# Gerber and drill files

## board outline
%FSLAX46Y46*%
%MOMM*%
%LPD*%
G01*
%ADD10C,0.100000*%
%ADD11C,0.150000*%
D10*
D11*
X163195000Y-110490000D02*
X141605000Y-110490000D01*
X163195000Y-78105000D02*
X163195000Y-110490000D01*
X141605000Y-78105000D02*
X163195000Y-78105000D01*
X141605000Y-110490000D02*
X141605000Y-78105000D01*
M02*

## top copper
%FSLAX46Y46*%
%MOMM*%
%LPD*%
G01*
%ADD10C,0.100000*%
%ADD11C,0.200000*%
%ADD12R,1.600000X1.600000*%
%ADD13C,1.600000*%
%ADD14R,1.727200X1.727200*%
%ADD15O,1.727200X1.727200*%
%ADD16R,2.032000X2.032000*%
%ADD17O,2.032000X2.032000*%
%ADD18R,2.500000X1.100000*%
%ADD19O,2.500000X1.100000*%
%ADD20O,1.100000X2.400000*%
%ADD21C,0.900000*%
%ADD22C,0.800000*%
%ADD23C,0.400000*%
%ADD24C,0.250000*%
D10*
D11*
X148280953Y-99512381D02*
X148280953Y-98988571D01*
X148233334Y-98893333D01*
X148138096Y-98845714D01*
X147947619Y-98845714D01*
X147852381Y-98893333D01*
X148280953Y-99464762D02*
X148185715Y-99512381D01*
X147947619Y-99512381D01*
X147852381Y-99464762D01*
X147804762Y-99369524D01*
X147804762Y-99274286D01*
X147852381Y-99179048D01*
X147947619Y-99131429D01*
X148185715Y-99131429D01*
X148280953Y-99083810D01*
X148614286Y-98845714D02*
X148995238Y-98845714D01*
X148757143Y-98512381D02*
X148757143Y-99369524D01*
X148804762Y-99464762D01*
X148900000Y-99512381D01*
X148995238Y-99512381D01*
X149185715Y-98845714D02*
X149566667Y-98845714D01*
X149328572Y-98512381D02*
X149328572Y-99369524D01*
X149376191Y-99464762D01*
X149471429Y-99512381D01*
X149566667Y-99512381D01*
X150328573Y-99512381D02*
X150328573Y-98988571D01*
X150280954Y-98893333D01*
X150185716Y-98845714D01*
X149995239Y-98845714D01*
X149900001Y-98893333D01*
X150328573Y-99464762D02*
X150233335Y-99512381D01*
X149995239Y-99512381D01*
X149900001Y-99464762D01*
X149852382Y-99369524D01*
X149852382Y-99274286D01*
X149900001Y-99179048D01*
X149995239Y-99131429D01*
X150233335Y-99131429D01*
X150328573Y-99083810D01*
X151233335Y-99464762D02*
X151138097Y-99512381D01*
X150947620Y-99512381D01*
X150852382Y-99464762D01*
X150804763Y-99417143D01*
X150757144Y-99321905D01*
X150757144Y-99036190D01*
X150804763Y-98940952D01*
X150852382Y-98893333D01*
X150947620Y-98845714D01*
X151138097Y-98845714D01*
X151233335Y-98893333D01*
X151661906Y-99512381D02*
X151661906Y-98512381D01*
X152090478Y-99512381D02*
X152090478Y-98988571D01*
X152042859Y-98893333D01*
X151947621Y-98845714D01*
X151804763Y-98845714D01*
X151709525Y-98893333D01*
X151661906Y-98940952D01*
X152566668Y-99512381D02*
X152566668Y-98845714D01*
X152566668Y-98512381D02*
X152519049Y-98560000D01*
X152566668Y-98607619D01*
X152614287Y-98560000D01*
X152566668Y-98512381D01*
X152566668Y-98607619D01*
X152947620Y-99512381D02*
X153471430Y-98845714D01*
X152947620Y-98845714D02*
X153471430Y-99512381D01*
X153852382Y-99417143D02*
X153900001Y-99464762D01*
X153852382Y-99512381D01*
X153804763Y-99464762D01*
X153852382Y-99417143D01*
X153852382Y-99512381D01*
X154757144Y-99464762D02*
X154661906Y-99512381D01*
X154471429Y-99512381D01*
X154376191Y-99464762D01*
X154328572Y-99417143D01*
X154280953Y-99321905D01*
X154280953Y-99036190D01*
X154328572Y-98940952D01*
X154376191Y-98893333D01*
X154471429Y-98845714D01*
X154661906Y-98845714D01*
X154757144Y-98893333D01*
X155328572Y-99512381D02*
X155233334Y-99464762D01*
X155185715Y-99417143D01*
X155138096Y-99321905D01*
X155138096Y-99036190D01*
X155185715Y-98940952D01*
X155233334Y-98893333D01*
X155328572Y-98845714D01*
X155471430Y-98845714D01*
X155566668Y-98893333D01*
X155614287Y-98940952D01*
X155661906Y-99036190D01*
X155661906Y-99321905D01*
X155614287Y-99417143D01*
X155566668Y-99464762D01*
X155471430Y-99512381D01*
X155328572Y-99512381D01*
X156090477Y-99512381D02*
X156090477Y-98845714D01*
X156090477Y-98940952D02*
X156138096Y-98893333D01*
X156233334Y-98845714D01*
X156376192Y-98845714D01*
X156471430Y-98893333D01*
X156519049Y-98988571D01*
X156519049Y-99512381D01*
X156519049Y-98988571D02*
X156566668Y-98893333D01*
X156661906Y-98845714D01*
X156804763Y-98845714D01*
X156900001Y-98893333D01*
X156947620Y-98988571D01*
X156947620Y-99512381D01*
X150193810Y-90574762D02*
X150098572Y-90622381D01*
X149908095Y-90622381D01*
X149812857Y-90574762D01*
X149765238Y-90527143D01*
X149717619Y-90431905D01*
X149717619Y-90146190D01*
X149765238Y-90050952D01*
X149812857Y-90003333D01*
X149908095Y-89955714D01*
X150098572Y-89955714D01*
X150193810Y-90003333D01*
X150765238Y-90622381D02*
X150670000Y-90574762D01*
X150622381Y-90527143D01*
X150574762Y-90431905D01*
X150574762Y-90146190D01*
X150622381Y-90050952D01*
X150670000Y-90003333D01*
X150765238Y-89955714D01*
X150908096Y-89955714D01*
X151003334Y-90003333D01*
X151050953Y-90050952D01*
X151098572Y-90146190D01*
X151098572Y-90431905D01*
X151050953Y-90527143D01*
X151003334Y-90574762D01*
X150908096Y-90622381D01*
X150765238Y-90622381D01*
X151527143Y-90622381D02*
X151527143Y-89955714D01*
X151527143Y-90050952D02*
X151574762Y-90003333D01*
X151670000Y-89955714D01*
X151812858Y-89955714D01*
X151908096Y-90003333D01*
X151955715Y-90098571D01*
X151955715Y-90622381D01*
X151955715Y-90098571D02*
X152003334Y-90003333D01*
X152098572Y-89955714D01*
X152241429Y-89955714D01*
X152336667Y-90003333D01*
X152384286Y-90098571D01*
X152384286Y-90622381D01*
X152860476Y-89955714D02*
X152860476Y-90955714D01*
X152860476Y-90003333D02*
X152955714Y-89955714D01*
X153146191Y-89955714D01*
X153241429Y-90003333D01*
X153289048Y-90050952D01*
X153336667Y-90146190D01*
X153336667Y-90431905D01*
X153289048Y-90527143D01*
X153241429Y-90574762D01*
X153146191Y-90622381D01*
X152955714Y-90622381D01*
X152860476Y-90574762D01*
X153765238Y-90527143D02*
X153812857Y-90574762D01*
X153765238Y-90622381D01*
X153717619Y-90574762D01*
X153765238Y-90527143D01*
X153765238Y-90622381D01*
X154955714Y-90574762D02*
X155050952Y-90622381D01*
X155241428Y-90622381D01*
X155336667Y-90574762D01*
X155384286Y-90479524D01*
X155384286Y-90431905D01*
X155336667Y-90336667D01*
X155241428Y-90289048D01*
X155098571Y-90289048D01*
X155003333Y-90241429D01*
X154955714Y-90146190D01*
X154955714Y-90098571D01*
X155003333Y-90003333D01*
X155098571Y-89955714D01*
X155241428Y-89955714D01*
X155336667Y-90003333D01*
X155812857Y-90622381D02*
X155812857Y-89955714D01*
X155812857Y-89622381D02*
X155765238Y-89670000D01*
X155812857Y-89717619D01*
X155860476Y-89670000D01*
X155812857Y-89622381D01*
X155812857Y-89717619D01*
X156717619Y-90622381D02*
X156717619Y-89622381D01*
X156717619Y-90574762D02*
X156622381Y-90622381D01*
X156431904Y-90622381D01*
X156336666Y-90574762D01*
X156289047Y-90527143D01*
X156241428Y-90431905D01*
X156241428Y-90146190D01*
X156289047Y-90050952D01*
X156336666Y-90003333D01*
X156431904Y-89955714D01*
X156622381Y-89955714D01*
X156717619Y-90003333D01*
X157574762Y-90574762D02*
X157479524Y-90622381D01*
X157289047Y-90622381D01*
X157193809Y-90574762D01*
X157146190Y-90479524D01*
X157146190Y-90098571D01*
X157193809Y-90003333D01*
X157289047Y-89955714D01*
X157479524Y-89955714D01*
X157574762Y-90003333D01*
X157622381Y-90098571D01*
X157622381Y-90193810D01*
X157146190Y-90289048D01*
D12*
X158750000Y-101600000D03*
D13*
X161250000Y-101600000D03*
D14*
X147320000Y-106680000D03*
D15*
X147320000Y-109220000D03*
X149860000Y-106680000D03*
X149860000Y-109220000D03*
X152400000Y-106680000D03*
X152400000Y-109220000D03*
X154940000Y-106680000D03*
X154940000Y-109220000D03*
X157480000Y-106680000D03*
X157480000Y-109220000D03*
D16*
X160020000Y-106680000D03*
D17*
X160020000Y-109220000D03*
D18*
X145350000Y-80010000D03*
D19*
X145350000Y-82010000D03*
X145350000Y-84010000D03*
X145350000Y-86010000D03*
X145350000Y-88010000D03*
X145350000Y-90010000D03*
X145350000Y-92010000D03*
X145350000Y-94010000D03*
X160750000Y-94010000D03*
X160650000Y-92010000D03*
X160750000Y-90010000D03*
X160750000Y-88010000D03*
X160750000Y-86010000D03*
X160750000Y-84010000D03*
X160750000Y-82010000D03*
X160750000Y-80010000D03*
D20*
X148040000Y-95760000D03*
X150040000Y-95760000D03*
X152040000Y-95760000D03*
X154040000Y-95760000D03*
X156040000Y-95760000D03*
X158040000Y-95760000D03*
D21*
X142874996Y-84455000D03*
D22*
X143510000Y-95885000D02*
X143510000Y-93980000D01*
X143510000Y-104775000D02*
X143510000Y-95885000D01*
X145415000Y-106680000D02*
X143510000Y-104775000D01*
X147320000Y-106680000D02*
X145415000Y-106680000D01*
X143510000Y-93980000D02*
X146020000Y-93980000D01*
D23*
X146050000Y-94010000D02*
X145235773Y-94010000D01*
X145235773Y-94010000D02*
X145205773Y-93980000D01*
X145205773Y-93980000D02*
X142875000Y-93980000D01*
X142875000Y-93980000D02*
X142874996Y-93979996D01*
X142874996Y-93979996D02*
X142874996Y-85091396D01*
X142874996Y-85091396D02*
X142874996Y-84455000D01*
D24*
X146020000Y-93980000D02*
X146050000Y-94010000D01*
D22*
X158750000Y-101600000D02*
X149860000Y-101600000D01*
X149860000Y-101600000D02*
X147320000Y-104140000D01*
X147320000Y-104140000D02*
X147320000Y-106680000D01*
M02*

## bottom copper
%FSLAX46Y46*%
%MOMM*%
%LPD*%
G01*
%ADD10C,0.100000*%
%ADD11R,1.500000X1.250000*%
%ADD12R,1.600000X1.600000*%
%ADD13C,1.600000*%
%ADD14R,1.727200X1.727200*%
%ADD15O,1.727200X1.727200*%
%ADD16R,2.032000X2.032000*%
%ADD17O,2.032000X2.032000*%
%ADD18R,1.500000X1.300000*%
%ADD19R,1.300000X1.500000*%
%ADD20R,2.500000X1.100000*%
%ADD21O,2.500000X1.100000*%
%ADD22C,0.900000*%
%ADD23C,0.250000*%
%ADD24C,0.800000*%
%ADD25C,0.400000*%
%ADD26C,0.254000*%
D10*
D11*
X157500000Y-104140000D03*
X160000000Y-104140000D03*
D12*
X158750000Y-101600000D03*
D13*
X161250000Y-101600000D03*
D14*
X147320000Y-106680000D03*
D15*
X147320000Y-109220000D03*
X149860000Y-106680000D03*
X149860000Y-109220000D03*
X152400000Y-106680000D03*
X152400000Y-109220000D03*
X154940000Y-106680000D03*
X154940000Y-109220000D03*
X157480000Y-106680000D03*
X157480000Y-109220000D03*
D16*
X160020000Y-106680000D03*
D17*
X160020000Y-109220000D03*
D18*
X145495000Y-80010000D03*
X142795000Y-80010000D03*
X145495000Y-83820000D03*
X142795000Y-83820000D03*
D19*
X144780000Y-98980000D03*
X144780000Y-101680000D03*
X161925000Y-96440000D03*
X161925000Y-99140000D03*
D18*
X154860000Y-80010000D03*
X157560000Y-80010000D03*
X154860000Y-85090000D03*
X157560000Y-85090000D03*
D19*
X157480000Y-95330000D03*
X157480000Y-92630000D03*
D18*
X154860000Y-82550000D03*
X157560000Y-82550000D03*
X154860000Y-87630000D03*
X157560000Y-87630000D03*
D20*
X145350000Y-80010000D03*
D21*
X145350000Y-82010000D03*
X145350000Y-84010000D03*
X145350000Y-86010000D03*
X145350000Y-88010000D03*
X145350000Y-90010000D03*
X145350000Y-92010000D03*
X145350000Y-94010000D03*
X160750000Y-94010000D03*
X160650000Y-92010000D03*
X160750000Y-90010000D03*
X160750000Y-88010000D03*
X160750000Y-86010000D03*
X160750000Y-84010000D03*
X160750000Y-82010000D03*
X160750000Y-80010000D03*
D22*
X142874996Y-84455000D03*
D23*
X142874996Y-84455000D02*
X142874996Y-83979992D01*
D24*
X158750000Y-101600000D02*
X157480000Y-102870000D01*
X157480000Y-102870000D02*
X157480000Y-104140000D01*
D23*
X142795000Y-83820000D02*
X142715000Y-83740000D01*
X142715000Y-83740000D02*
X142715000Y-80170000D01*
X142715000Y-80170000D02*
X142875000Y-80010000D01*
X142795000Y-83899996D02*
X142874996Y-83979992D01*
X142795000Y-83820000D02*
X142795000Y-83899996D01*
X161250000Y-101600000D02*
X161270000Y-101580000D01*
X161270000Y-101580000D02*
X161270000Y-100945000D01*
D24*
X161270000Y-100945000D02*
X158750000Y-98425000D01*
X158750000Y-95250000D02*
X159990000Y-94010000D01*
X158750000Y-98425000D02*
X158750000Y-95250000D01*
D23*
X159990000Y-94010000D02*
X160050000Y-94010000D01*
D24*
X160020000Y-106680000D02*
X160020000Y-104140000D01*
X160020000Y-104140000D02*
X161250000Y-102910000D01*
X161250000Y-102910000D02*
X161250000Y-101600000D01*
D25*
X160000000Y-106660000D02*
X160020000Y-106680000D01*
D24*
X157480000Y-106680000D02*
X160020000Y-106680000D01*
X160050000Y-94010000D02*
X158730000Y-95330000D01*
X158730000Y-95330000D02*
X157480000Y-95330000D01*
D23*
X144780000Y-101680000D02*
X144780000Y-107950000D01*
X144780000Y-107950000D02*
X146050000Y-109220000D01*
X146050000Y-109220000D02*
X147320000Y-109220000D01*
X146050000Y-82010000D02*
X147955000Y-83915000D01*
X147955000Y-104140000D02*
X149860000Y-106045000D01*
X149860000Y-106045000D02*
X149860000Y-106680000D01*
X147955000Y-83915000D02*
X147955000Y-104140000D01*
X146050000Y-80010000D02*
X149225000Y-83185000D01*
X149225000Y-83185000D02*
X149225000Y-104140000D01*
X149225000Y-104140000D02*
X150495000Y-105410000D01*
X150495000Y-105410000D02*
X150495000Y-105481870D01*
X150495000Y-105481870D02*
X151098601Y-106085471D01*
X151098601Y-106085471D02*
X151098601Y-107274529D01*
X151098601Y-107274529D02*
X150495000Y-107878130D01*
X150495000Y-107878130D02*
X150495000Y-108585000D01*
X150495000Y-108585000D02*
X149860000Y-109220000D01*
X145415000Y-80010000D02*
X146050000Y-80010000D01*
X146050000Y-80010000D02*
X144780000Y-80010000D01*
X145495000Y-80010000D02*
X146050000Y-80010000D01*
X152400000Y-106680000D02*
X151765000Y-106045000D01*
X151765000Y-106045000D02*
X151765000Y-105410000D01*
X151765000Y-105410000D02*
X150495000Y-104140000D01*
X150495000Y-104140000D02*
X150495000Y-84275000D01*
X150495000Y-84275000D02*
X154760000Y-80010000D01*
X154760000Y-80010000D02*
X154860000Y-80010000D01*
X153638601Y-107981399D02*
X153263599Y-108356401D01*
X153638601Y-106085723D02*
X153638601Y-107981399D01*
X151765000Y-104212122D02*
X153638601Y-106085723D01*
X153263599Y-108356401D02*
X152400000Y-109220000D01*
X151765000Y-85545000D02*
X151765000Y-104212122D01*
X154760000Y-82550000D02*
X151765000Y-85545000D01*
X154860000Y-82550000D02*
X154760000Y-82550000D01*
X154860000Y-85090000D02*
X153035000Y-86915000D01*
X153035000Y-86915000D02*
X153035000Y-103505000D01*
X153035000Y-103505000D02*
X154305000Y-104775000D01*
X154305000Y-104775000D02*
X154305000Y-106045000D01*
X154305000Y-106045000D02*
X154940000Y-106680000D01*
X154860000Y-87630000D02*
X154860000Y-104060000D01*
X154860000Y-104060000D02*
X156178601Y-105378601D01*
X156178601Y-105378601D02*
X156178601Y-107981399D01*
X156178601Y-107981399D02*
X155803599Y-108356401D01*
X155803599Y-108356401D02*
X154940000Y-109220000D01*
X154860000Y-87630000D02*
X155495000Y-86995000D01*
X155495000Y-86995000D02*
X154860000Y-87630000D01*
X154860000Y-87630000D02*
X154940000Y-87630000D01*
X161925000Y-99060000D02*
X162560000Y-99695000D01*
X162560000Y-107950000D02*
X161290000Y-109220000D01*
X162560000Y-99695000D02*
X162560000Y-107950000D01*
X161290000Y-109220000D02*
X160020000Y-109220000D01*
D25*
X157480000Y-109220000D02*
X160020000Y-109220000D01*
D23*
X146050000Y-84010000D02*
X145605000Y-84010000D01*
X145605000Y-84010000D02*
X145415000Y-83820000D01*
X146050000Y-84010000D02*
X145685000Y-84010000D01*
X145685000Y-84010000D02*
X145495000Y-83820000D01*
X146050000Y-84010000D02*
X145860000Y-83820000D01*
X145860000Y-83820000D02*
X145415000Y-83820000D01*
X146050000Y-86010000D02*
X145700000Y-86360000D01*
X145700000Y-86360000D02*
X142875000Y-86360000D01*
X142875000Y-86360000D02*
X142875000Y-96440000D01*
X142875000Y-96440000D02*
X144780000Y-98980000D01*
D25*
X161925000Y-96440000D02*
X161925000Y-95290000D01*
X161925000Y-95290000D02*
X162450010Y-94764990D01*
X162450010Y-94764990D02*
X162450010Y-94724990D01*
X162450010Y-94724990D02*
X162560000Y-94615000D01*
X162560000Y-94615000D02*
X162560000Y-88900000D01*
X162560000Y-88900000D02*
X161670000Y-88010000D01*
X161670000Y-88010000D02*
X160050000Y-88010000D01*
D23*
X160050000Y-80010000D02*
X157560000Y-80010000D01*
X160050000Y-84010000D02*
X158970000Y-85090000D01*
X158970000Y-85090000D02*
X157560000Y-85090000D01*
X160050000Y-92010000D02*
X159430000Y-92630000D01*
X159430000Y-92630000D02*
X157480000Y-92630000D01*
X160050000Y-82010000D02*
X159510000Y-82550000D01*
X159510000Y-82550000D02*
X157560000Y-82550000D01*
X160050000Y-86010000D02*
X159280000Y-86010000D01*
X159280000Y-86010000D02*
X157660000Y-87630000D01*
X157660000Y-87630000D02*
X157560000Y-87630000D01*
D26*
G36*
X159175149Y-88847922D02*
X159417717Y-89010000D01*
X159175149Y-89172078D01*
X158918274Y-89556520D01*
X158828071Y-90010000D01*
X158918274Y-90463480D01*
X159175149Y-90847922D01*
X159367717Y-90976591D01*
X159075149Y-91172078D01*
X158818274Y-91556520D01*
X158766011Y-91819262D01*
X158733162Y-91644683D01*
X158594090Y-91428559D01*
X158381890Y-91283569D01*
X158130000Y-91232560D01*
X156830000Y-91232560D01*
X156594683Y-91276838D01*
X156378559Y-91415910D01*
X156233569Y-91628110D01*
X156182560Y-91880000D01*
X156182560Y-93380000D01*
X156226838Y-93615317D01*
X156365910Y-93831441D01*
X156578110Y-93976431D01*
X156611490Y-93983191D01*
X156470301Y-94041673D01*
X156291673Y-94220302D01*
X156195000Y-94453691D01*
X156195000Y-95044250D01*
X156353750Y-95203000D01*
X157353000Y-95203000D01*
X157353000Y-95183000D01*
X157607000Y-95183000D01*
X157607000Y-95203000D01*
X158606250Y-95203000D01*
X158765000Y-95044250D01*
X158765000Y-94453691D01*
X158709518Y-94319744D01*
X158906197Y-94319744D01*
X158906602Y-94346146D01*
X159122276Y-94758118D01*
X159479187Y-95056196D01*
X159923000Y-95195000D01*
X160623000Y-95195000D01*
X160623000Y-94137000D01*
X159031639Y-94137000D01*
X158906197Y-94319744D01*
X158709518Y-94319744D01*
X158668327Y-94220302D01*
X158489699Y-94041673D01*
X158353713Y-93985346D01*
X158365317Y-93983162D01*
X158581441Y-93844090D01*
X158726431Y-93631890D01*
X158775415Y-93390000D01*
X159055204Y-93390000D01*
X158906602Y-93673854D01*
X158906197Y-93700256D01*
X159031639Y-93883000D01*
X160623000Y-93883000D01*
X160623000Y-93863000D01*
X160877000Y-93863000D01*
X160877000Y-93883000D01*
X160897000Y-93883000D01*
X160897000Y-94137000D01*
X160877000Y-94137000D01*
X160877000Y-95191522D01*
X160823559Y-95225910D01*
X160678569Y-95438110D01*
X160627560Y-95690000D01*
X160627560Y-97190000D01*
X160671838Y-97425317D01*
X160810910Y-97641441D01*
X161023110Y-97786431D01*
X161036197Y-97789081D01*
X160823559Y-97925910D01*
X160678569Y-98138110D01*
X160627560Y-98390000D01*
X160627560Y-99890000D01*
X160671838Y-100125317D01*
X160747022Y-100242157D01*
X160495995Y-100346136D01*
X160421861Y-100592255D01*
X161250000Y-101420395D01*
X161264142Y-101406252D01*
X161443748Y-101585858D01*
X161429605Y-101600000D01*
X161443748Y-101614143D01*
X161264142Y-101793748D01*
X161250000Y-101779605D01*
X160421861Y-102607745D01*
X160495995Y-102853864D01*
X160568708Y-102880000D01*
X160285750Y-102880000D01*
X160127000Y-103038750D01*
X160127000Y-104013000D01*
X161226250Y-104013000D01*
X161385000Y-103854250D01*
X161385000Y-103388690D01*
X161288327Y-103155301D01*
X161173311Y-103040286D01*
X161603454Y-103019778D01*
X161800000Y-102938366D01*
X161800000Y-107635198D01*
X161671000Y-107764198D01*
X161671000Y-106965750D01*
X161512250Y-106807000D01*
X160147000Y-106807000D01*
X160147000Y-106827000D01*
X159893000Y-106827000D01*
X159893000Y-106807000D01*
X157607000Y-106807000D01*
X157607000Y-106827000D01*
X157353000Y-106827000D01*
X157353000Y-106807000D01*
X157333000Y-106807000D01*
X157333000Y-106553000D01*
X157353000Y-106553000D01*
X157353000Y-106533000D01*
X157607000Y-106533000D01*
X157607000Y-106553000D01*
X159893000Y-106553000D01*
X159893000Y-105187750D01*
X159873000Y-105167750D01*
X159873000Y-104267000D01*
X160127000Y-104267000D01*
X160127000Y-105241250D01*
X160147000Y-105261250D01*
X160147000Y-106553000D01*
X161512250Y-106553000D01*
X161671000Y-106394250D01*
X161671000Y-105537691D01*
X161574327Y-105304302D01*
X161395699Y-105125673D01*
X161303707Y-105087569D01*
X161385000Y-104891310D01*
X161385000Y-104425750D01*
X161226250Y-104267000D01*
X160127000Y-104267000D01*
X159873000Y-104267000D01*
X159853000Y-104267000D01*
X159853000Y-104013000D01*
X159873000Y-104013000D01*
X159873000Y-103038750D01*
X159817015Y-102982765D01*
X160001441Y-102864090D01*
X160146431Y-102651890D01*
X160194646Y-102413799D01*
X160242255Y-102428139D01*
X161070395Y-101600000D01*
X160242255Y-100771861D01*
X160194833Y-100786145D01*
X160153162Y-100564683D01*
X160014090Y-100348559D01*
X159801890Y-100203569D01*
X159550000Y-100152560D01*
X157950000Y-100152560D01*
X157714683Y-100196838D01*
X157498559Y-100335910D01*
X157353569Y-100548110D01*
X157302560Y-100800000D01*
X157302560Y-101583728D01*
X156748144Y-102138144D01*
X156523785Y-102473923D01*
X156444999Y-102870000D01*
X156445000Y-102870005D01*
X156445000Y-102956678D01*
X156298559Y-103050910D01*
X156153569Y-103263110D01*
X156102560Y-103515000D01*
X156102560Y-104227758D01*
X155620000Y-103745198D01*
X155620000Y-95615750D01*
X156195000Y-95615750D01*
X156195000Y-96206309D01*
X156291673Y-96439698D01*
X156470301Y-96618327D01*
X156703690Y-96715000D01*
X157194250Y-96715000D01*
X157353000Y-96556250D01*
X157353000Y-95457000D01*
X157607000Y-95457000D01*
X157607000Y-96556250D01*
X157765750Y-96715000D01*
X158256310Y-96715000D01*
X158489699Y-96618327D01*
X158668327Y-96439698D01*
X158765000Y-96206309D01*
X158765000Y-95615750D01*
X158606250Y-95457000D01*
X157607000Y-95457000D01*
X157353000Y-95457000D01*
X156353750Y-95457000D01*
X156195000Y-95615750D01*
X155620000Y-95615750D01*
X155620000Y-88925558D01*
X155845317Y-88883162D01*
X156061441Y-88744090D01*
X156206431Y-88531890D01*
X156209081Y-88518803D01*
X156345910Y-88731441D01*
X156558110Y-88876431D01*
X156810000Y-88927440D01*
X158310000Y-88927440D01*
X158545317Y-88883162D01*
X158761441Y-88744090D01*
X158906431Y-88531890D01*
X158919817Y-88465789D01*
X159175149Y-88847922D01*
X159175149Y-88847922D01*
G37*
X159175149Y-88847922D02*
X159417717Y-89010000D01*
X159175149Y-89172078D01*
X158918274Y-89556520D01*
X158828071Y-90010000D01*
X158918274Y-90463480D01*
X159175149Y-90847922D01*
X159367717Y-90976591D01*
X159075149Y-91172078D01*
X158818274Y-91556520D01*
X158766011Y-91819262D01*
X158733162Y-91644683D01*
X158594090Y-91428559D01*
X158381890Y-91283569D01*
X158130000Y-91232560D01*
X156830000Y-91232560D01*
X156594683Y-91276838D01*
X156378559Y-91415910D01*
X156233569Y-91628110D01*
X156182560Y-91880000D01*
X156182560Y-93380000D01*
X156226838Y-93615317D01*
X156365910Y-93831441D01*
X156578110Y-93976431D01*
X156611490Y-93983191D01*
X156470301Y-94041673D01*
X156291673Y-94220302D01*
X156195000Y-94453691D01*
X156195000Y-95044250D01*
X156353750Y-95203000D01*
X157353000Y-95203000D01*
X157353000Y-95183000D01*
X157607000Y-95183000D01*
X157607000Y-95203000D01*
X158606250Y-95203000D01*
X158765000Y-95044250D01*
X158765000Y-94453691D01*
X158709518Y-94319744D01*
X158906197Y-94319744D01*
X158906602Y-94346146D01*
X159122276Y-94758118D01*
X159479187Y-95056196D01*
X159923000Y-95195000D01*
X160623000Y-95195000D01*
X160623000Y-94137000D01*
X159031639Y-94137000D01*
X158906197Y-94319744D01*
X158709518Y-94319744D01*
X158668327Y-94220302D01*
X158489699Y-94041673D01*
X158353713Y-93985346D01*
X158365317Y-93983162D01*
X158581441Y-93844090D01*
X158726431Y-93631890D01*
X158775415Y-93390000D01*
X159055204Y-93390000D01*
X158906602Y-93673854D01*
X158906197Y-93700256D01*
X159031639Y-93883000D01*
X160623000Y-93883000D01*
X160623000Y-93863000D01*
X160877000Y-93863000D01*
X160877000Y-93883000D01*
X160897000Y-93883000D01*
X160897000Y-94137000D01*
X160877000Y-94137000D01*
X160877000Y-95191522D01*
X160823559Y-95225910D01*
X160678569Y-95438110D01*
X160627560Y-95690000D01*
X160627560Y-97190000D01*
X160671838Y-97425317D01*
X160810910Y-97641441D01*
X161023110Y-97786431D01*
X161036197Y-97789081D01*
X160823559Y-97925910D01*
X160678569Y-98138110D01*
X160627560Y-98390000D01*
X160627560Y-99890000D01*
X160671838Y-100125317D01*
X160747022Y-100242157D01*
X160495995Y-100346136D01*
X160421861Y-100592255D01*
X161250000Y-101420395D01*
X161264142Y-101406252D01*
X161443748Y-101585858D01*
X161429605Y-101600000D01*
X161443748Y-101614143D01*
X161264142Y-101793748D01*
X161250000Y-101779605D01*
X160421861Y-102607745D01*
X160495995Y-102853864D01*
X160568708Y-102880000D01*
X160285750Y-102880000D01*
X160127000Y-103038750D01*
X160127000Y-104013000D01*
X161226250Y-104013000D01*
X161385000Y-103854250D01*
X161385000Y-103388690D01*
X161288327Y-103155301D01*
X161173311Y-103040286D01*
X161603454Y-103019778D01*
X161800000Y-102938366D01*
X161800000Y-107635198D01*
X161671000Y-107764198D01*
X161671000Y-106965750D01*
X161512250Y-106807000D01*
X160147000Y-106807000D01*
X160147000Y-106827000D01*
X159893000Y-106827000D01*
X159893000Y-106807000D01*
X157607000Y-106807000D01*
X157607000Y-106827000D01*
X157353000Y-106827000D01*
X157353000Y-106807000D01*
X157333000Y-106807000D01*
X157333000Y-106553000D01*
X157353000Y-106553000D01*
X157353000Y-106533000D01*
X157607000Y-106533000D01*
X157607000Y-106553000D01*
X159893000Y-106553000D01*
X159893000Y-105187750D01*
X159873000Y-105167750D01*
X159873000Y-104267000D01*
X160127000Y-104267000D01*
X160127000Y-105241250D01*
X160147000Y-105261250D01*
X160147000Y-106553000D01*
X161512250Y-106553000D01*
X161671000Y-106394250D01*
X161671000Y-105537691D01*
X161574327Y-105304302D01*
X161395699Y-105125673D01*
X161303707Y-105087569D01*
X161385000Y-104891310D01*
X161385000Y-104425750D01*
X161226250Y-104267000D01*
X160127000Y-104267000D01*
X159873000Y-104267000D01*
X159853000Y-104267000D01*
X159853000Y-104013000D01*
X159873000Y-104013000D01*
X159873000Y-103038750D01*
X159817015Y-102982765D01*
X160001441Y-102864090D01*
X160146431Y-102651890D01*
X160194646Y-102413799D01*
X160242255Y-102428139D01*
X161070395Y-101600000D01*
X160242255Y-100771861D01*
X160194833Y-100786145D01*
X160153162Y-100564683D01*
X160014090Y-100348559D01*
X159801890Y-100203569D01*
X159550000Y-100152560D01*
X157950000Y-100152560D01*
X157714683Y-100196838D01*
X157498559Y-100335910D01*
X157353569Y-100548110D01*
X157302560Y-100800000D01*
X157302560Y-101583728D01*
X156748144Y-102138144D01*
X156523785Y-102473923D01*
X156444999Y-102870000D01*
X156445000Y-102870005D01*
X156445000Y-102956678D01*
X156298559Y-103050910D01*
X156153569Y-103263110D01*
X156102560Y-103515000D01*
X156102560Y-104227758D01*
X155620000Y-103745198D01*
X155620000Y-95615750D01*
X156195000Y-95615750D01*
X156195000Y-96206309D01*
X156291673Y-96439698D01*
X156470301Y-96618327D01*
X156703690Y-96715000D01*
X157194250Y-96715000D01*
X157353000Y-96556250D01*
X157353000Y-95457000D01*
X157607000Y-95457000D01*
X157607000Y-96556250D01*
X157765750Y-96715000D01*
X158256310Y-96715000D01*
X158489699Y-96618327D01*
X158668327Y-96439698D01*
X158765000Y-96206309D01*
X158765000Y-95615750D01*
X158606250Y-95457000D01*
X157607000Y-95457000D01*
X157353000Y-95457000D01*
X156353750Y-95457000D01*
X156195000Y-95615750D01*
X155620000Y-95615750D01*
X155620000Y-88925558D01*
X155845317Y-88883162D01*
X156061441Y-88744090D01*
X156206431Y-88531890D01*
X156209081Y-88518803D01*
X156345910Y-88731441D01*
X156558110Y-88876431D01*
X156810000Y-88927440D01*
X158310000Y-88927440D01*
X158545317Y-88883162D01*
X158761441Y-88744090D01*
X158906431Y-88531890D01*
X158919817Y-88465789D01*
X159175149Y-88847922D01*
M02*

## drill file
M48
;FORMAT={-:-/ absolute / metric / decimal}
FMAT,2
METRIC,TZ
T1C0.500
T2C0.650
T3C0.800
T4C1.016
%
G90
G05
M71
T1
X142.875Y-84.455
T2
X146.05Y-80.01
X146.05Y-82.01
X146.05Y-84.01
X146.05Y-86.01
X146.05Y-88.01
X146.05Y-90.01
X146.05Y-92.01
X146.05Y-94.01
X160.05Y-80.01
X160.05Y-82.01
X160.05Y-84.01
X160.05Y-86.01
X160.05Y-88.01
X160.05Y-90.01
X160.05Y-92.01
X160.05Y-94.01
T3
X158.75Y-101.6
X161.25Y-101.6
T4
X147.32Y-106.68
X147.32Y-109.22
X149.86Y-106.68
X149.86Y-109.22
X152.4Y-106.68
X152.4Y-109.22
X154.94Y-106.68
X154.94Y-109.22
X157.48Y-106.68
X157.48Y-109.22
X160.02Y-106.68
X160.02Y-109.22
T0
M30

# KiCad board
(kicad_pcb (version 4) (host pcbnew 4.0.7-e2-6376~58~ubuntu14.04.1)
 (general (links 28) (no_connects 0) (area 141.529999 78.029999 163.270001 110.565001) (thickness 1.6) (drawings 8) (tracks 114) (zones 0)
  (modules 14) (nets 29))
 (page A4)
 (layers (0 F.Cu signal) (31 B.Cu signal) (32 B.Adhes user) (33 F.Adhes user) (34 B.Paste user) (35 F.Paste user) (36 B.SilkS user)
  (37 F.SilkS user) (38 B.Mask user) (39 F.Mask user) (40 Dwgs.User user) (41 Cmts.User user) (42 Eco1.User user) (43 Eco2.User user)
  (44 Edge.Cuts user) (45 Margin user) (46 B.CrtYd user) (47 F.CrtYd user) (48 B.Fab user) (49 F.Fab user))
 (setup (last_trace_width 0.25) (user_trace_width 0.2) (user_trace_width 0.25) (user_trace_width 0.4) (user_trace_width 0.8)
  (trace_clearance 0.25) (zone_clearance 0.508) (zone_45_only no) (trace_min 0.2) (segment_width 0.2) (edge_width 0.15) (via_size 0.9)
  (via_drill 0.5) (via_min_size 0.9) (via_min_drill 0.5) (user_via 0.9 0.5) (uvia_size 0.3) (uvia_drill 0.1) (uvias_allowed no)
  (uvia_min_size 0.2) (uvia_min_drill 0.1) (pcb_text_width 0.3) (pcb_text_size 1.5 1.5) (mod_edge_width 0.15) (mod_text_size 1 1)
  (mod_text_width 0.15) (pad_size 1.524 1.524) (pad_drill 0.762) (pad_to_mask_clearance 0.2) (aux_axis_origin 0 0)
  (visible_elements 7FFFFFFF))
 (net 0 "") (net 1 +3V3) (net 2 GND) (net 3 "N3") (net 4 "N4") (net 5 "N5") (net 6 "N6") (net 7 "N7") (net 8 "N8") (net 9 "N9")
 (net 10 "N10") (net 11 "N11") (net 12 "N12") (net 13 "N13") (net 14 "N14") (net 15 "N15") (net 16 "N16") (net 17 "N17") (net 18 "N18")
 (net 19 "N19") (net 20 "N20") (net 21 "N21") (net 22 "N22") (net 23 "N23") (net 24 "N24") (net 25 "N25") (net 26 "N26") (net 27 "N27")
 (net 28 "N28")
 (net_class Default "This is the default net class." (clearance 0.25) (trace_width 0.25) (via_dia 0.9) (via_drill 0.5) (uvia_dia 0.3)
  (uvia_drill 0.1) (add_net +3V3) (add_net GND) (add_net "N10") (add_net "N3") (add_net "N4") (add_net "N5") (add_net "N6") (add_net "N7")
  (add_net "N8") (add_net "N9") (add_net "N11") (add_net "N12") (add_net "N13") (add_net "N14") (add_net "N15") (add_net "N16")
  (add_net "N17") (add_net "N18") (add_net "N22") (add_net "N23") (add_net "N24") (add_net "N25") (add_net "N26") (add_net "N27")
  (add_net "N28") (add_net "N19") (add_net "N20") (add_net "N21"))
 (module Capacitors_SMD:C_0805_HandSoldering (layer B.Cu) (at 158.75 104.14)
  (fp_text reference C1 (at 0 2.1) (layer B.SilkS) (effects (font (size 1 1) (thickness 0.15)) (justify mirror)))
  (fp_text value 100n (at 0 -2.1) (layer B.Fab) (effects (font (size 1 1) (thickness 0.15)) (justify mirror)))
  (pad 1 smd rect (at -1.25 0) (size 1.5 1.25) (layers B.Cu B.Paste B.Mask) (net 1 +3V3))
  (pad 2 smd rect (at 1.25 0) (size 1.5 1.25) (layers B.Cu B.Paste B.Mask) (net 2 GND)))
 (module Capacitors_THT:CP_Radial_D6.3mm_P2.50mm (layer F.Cu) (at 158.75 101.6)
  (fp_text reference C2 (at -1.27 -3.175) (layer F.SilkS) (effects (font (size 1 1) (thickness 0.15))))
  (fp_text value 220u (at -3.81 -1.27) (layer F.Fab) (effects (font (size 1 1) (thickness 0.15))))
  (pad 1 thru_hole rect (at 0 0) (size 1.6 1.6) (drill 0.8) (layers *.Cu *.Mask) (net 1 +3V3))
  (pad 2 thru_hole circle (at 2.5 0) (size 1.6 1.6) (drill 0.8) (layers *.Cu *.Mask) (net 2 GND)))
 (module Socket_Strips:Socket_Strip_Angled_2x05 (layer F.Cu) (at 147.32 106.68)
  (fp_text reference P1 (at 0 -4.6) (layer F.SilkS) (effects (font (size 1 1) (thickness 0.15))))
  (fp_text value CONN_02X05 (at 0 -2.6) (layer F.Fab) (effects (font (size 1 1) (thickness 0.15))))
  (pad 1 thru_hole rect (at 0 0) (size 1.7272 1.7272) (drill 1.016) (layers *.Cu *.Mask) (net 1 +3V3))
  (pad 2 thru_hole oval (at 0 2.54) (size 1.7272 1.7272) (drill 1.016) (layers *.Cu *.Mask) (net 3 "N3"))
  (pad 3 thru_hole oval (at 2.54 0) (size 1.7272 1.7272) (drill 1.016) (layers *.Cu *.Mask) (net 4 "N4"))
  (pad 4 thru_hole oval (at 2.54 2.54) (size 1.7272 1.7272) (drill 1.016) (layers *.Cu *.Mask) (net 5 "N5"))
  (pad 5 thru_hole oval (at 5.08 0) (size 1.7272 1.7272) (drill 1.016) (layers *.Cu *.Mask) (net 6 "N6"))
  (pad 6 thru_hole oval (at 5.08 2.54) (size 1.7272 1.7272) (drill 1.016) (layers *.Cu *.Mask) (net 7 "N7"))
  (pad 7 thru_hole oval (at 7.62 0) (size 1.7272 1.7272) (drill 1.016) (layers *.Cu *.Mask) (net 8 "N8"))
  (pad 8 thru_hole oval (at 7.62 2.54) (size 1.7272 1.7272) (drill 1.016) (layers *.Cu *.Mask) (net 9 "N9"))
  (pad 9 thru_hole oval (at 10.16 0) (size 1.7272 1.7272) (drill 1.016) (layers *.Cu *.Mask) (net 2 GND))
  (pad 10 thru_hole oval (at 10.16 2.54) (size 1.7272 1.7272) (drill 1.016) (layers *.Cu *.Mask) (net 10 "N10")))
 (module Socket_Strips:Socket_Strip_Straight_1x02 (layer F.Cu) (at 160.02 106.68 270)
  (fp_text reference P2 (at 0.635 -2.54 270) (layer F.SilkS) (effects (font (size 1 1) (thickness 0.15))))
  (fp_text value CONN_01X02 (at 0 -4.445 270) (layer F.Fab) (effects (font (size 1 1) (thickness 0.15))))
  (pad 1 thru_hole rect (at 0 0 270) (size 2.032 2.032) (drill 1.016) (layers *.Cu *.Mask) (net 2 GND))
  (pad 2 thru_hole oval (at 2.54 0 270) (size 2.032 2.032) (drill 1.016) (layers *.Cu *.Mask) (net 10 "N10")))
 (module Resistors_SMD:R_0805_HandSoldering (layer B.Cu) (at 144.145 80.01 180)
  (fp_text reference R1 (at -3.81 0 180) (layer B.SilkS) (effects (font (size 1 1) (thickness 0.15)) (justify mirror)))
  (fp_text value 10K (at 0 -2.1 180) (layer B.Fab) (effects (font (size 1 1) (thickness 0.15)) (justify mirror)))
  (pad 1 smd rect (at -1.35 0 180) (size 1.5 1.3) (layers B.Cu B.Paste B.Mask) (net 5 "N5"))
  (pad 2 smd rect (at 1.35 0 180) (size 1.5 1.3) (layers B.Cu B.Paste B.Mask) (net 1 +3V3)))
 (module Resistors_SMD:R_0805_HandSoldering (layer B.Cu) (at 144.145 83.82 180)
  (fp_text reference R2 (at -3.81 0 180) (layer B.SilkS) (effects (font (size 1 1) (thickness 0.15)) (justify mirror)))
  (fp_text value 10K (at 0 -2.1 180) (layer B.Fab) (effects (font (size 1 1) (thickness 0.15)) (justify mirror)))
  (pad 1 smd rect (at -1.35 0 180) (size 1.5 1.3) (layers B.Cu B.Paste B.Mask) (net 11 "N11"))
  (pad 2 smd rect (at 1.35 0 180) (size 1.5 1.3) (layers B.Cu B.Paste B.Mask) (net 1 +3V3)))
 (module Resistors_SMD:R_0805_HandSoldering (layer B.Cu) (at 144.78 100.33 270)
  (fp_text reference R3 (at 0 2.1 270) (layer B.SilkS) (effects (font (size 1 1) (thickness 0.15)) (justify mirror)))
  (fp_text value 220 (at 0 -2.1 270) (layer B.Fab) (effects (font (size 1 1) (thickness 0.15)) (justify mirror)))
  (pad 1 smd rect (at -1.35 0 270) (size 1.5 1.3) (layers B.Cu B.Paste B.Mask) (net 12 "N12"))
  (pad 2 smd rect (at 1.35 0 270) (size 1.5 1.3) (layers B.Cu B.Paste B.Mask) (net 3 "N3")))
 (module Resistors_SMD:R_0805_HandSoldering (layer B.Cu) (at 161.925 97.79 270)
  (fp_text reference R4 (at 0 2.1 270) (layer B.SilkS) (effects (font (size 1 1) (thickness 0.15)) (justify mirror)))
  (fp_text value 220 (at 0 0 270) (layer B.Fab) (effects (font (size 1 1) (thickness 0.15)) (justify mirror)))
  (pad 1 smd rect (at -1.35 0 270) (size 1.5 1.3) (layers B.Cu B.Paste B.Mask) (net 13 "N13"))
  (pad 2 smd rect (at 1.35 0 270) (size 1.5 1.3) (layers B.Cu B.Paste B.Mask) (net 10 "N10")))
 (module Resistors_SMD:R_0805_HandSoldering (layer B.Cu) (at 156.21 80.01)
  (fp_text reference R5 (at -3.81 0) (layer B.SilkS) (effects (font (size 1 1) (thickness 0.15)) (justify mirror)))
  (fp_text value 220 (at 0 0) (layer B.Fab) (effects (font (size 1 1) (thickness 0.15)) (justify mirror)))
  (pad 1 smd rect (at -1.35 0) (size 1.5 1.3) (layers B.Cu B.Paste B.Mask) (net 6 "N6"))
  (pad 2 smd rect (at 1.35 0) (size 1.5 1.3) (layers B.Cu B.Paste B.Mask) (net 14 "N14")))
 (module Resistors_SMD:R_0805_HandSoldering (layer B.Cu) (at 156.21 85.09)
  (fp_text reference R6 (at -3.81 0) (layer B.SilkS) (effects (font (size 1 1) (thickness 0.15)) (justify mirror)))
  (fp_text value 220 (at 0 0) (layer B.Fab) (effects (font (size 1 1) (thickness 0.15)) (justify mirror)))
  (pad 1 smd rect (at -1.35 0) (size 1.5 1.3) (layers B.Cu B.Paste B.Mask) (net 8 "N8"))
  (pad 2 smd rect (at 1.35 0) (size 1.5 1.3) (layers B.Cu B.Paste B.Mask) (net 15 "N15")))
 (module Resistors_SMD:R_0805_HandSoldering (layer B.Cu) (at 157.48 93.98 90)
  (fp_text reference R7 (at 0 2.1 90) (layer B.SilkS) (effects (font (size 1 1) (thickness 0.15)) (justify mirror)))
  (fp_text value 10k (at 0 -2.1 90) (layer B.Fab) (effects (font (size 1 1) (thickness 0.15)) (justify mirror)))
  (pad 1 smd rect (at -1.35 0 90) (size 1.5 1.3) (layers B.Cu B.Paste B.Mask) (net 2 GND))
  (pad 2 smd rect (at 1.35 0 90) (size 1.5 1.3) (layers B.Cu B.Paste B.Mask) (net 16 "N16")))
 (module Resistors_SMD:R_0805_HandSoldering (layer B.Cu) (at 156.21 82.55)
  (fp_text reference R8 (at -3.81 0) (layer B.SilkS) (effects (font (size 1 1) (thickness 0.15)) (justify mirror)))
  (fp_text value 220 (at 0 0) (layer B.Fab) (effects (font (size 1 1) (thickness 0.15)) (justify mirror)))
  (pad 1 smd rect (at -1.35 0) (size 1.5 1.3) (layers B.Cu B.Paste B.Mask) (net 7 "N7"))
  (pad 2 smd rect (at 1.35 0) (size 1.5 1.3) (layers B.Cu B.Paste B.Mask) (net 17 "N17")))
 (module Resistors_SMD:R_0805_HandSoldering (layer B.Cu) (at 156.21 87.63)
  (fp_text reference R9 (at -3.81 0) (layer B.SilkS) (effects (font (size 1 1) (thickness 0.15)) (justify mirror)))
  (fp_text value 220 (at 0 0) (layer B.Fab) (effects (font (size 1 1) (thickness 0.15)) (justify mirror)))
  (pad 1 smd rect (at -1.35 0) (size 1.5 1.3) (layers B.Cu B.Paste B.Mask) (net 9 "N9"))
  (pad 2 smd rect (at 1.35 0) (size 1.5 1.3) (layers B.Cu B.Paste B.Mask) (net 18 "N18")))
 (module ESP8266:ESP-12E (layer F.Cu) (at 146.05 80.01)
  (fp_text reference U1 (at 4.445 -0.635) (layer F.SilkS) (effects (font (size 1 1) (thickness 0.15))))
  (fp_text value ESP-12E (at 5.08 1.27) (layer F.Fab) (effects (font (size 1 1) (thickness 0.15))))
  (pad 1 thru_hole rect (at 0 0) (size 2.5 1.1) (drill 0.65 (offset -0.7 0)) (layers *.Cu *.Mask F.SilkS) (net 5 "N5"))
  (pad 2 thru_hole oval (at 0 2) (size 2.5 1.1) (drill 0.65 (offset -0.7 0)) (layers *.Cu *.Mask F.SilkS) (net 4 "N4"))
  (pad 3 thru_hole oval (at 0 4) (size 2.5 1.1) (drill 0.65 (offset -0.7 0)) (layers *.Cu *.Mask F.SilkS) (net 11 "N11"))
  (pad 4 thru_hole oval (at 0 6) (size 2.5 1.1) (drill 0.65 (offset -0.7 0)) (layers *.Cu *.Mask F.SilkS) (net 12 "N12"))
  (pad 5 thru_hole oval (at 0 8) (size 2.5 1.1) (drill 0.65 (offset -0.7 0)) (layers *.Cu *.Mask F.SilkS) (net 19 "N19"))
  (pad 6 thru_hole oval (at 0 10) (size 2.5 1.1) (drill 0.65 (offset -0.7 0)) (layers *.Cu *.Mask F.SilkS) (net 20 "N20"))
  (pad 7 thru_hole oval (at 0 12) (size 2.5 1.1) (drill 0.65 (offset -0.7 0)) (layers *.Cu *.Mask F.SilkS) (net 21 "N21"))
  (pad 8 thru_hole oval (at 0 14) (size 2.5 1.1) (drill 0.65 (offset -0.7 0)) (layers *.Cu *.Mask F.SilkS) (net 1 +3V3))
  (pad 9 thru_hole oval (at 14 14) (size 2.5 1.1) (drill 0.65 (offset 0.7 0)) (layers *.Cu *.Mask F.SilkS) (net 2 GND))
  (pad 10 thru_hole oval (at 14 12) (size 2.5 1.1) (drill 0.65 (offset 0.6 0)) (layers *.Cu *.Mask F.SilkS) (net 16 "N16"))
  (pad 11 thru_hole oval (at 14 10) (size 2.5 1.1) (drill 0.65 (offset 0.7 0)) (layers *.Cu *.Mask F.SilkS) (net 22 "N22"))
  (pad 12 thru_hole oval (at 14 8) (size 2.5 1.1) (drill 0.65 (offset 0.7 0)) (layers *.Cu *.Mask F.SilkS) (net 13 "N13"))
  (pad 13 thru_hole oval (at 14 6) (size 2.5 1.1) (drill 0.65 (offset 0.7 0)) (layers *.Cu *.Mask F.SilkS) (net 18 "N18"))
  (pad 14 thru_hole oval (at 14 4) (size 2.5 1.1) (drill 0.65 (offset 0.7 0)) (layers *.Cu *.Mask F.SilkS) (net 15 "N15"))
  (pad 15 thru_hole oval (at 14 2) (size 2.5 1.1) (drill 0.65 (offset 0.7 0)) (layers *.Cu *.Mask F.SilkS) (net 17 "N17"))
  (pad 16 thru_hole oval (at 14 0) (size 2.5 1.1) (drill 0.65 (offset 0.7 0)) (layers *.Cu *.Mask F.SilkS) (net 14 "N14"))
  (pad 17 smd oval (at 1.99 15.75 90) (size 2.4 1.1) (layers F.Cu F.Paste F.Mask) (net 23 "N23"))
  (pad 18 smd oval (at 3.99 15.75 90) (size 2.4 1.1) (layers F.Cu F.Paste F.Mask) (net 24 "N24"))
  (pad 19 smd oval (at 5.99 15.75 90) (size 2.4 1.1) (layers F.Cu F.Paste F.Mask) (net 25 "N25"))
  (pad 20 smd oval (at 7.99 15.75 90) (size 2.4 1.1) (layers F.Cu F.Paste F.Mask) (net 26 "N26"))
  (pad 21 smd oval (at 9.99 15.75 90) (size 2.4 1.1) (layers F.Cu F.Paste F.Mask) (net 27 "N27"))
  (pad 22 smd oval (at 11.99 15.75 90) (size 2.4 1.1) (layers F.Cu F.Paste F.Mask) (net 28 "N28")))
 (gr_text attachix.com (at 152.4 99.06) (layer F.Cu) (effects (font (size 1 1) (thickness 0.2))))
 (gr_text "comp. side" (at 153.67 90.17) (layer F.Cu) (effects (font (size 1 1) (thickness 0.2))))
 (gr_line (start 163.195 110.49) (end 141.605 110.49) (angle 90) (layer Edge.Cuts) (width 0.15))
 (gr_line (start 163.195 78.105) (end 163.195 110.49) (angle 90) (layer Edge.Cuts) (width 0.15))
 (gr_line (start 141.605 78.105) (end 163.195 78.105) (angle 90) (layer Edge.Cuts) (width 0.15))
 (gr_line (start 141.605 110.49) (end 141.605 78.105) (angle 90) (layer Edge.Cuts) (width 0.15))
 (segment (start 143.51 95.885) (end 143.51 93.98) (width 0.8) (layer F.Cu) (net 1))
 (segment (start 143.51 104.775) (end 143.51 95.885) (width 0.8) (layer F.Cu) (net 1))
 (segment (start 145.415 106.68) (end 143.51 104.775) (width 0.8) (layer F.Cu) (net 1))
 (segment (start 147.32 106.68) (end 145.415 106.68) (width 0.8) (layer F.Cu) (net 1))
 (segment (start 143.51 93.98) (end 146.02 93.98) (width 0.8) (layer F.Cu) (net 1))
 (segment (start 146.05 94.01) (end 145.235773 94.01) (width 0.4) (layer F.Cu) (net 1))
 (segment (start 145.235773 94.01) (end 145.205773 93.98) (width 0.4) (layer F.Cu) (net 1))
 (segment (start 145.205773 93.98) (end 142.875 93.98) (width 0.4) (layer F.Cu) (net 1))
 (segment (start 142.875 93.98) (end 142.874996 93.979996) (width 0.4) (layer F.Cu) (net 1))
 (segment (start 142.874996 93.979996) (end 142.874996 85.091396) (width 0.4) (layer F.Cu) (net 1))
 (segment (start 142.874996 85.091396) (end 142.874996 84.455) (width 0.4) (layer F.Cu) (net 1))
 (segment (start 146.02 93.98) (end 146.05 94.01) (width 0.25) (layer F.Cu) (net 1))
 (via (at 142.874996 84.455) (size 0.9) (drill 0.5) (layers F.Cu B.Cu) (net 1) (status 30))
 (segment (start 142.874996 84.455) (end 142.874996 83.979992) (width 0.25) (layer B.Cu) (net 1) (status 30))
 (segment (start 158.75 101.6) (end 149.86 101.6) (width 0.8) (layer F.Cu) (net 1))
 (segment (start 149.86 101.6) (end 147.32 104.14) (width 0.8) (layer F.Cu) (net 1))
 (segment (start 147.32 104.14) (end 147.32 106.68) (width 0.8) (layer F.Cu) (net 1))
 (segment (start 158.75 101.6) (end 157.48 102.87) (width 0.8) (layer B.Cu) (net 1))
 (segment (start 157.48 102.87) (end 157.48 104.14) (width 0.8) (layer B.Cu) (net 1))
 (segment (start 142.795 83.82) (end 142.715 83.74) (width 0.25) (layer B.Cu) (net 1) (status 30))
 (segment (start 142.715 83.74) (end 142.715 80.17) (width 0.25) (layer B.Cu) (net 1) (status 20))
 (segment (start 142.715 80.17) (end 142.875 80.01) (width 0.25) (layer B.Cu) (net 1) (status 30))
 (segment (start 142.795 83.899996) (end 142.874996 83.979992) (width 0.25) (layer B.Cu) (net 1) (status 30))
 (segment (start 142.795 83.82) (end 142.795 83.899996) (width 0.25) (layer B.Cu) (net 1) (status 30))
 (segment (start 161.25 101.6) (end 161.27 101.58) (width 0.25) (layer B.Cu) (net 2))
 (segment (start 161.27 101.58) (end 161.27 100.945) (width 0.25) (layer B.Cu) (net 2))
 (segment (start 161.27 100.945) (end 158.75 98.425) (width 0.8) (layer B.Cu) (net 2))
 (segment (start 158.75 95.25) (end 159.99 94.01) (width 0.8) (layer B.Cu) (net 2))
 (segment (start 158.75 98.425) (end 158.75 95.25) (width 0.8) (layer B.Cu) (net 2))
 (segment (start 159.99 94.01) (end 160.05 94.01) (width 0.25) (layer B.Cu) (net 2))
 (segment (start 160.02 106.68) (end 160.02 104.14) (width 0.8) (layer B.Cu) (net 2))
 (segment (start 160.02 104.14) (end 161.25 102.91) (width 0.8) (layer B.Cu) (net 2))
 (segment (start 161.25 102.91) (end 161.25 101.6) (width 0.8) (layer B.Cu) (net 2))
 (segment (start 160 106.66) (end 160.02 106.68) (width 0.4) (layer B.Cu) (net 2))
 (segment (start 157.48 106.68) (end 160.02 106.68) (width 0.8) (layer B.Cu) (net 2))
 (segment (start 160.05 94.01) (end 158.73 95.33) (width 0.8) (layer B.Cu) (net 2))
 (segment (start 158.73 95.33) (end 157.48 95.33) (width 0.8) (layer B.Cu) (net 2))
 (segment (start 144.78 101.68) (end 144.78 107.95) (width 0.25) (layer B.Cu) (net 3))
 (segment (start 144.78 107.95) (end 146.05 109.22) (width 0.25) (layer B.Cu) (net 3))
 (segment (start 146.05 109.22) (end 147.32 109.22) (width 0.25) (layer B.Cu) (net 3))
 (segment (start 146.05 82.01) (end 147.955 83.915) (width 0.25) (layer B.Cu) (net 4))
 (segment (start 147.955 104.14) (end 149.86 106.045) (width 0.25) (layer B.Cu) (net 4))
 (segment (start 149.86 106.045) (end 149.86 106.68) (width 0.25) (layer B.Cu) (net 4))
 (segment (start 147.955 83.915) (end 147.955 104.14) (width 0.25) (layer B.Cu) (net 4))
 (segment (start 146.05 80.01) (end 149.225 83.185) (width 0.25) (layer B.Cu) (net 5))
 (segment (start 149.225 83.185) (end 149.225 104.14) (width 0.25) (layer B.Cu) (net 5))
 (segment (start 149.225 104.14) (end 150.495 105.41) (width 0.25) (layer B.Cu) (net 5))
 (segment (start 150.495 105.41) (end 150.495 105.48187) (width 0.25) (layer B.Cu) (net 5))
 (segment (start 150.495 105.48187) (end 151.098601 106.085471) (width 0.25) (layer B.Cu) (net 5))
 (segment (start 151.098601 106.085471) (end 151.098601 107.274529) (width 0.25) (layer B.Cu) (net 5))
 (segment (start 151.098601 107.274529) (end 150.495 107.87813) (width 0.25) (layer B.Cu) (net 5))
 (segment (start 150.495 107.87813) (end 150.495 108.585) (width 0.25) (layer B.Cu) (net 5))
 (segment (start 150.495 108.585) (end 149.86 109.22) (width 0.25) (layer B.Cu) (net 5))
 (segment (start 145.415 80.01) (end 146.05 80.01) (width 0.25) (layer B.Cu) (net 5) (status 10))
 (segment (start 146.05 80.01) (end 144.78 80.01) (width 0.25) (layer B.Cu) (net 5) (status 20))
 (segment (start 145.495 80.01) (end 146.05 80.01) (width 0.25) (layer B.Cu) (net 5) (status 10))
 (segment (start 152.4 106.68) (end 151.765 106.045) (width 0.25) (layer B.Cu) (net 6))
 (segment (start 151.765 106.045) (end 151.765 105.41) (width 0.25) (layer B.Cu) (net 6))
 (segment (start 151.765 105.41) (end 150.495 104.14) (width 0.25) (layer B.Cu) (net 6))
 (segment (start 150.495 104.14) (end 150.495 84.275) (width 0.25) (layer B.Cu) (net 6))
 (segment (start 150.495 84.275) (end 154.76 80.01) (width 0.25) (layer B.Cu) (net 6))
 (segment (start 154.76 80.01) (end 154.86 80.01) (width 0.25) (layer B.Cu) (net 6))
 (segment (start 153.638601 107.981399) (end 153.263599 108.356401) (width 0.25) (layer B.Cu) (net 7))
 (segment (start 153.638601 106.085723) (end 153.638601 107.981399) (width 0.25) (layer B.Cu) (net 7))
 (segment (start 151.765 104.212122) (end 153.638601 106.085723) (width 0.25) (layer B.Cu) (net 7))
 (segment (start 153.263599 108.356401) (end 152.4 109.22) (width 0.25) (layer B.Cu) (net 7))
 (segment (start 151.765 85.545) (end 151.765 104.212122) (width 0.25) (layer B.Cu) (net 7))
 (segment (start 154.76 82.55) (end 151.765 85.545) (width 0.25) (layer B.Cu) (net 7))
 (segment (start 154.86 82.55) (end 154.76 82.55) (width 0.25) (layer B.Cu) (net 7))
 (segment (start 154.86 85.09) (end 153.035 86.915) (width 0.25) (layer B.Cu) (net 8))
 (segment (start 153.035 86.915) (end 153.035 103.505) (width 0.25) (layer B.Cu) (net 8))
 (segment (start 153.035 103.505) (end 154.305 104.775) (width 0.25) (layer B.Cu) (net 8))
 (segment (start 154.305 104.775) (end 154.305 106.045) (width 0.25) (layer B.Cu) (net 8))
 (segment (start 154.305 106.045) (end 154.94 106.68) (width 0.25) (layer B.Cu) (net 8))
 (segment (start 154.86 87.63) (end 154.86 104.06) (width 0.25) (layer B.Cu) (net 9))
 (segment (start 154.86 104.06) (end 156.178601 105.378601) (width 0.25) (layer B.Cu) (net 9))
 (segment (start 156.178601 105.378601) (end 156.178601 107.981399) (width 0.25) (layer B.Cu) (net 9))
 (segment (start 156.178601 107.981399) (end 155.803599 108.356401) (width 0.25) (layer B.Cu) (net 9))
 (segment (start 155.803599 108.356401) (end 154.94 109.22) (width 0.25) (layer B.Cu) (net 9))
 (segment (start 154.86 87.63) (end 155.495 86.995) (width 0.25) (layer B.Cu) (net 9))
 (segment (start 155.495 86.995) (end 154.86 87.63) (width 0.25) (layer B.Cu) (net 9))
 (segment (start 154.86 87.63) (end 154.94 87.63) (width 0.25) (layer B.Cu) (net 9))
 (segment (start 161.925 99.06) (end 162.56 99.695) (width 0.25) (layer B.Cu) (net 10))
 (segment (start 162.56 107.95) (end 161.29 109.22) (width 0.25) (layer B.Cu) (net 10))
 (segment (start 162.56 99.695) (end 162.56 107.95) (width 0.25) (layer B.Cu) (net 10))
 (segment (start 161.29 109.22) (end 160.02 109.22) (width 0.25) (layer B.Cu) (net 10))
 (segment (start 157.48 109.22) (end 160.02 109.22) (width 0.4) (layer B.Cu) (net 10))
 (segment (start 146.05 84.01) (end 145.605 84.01) (width 0.25) (layer B.Cu) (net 11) (status 20))
 (segment (start 145.605 84.01) (end 145.415 83.82) (width 0.25) (layer B.Cu) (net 11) (status 30))
 (segment (start 146.05 84.01) (end 145.685 84.01) (width 0.25) (layer B.Cu) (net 11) (status 20))
 (segment (start 145.685 84.01) (end 145.495 83.82) (width 0.25) (layer B.Cu) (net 11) (status 30))
 (segment (start 146.05 84.01) (end 145.86 83.82) (width 0.25) (layer B.Cu) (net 11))
 (segment (start 145.86 83.82) (end 145.415 83.82) (width 0.25) (layer B.Cu) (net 11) (status 20))
 (segment (start 146.05 86.01) (end 145.7 86.36) (width 0.25) (layer B.Cu) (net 12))
 (segment (start 145.7 86.36) (end 142.875 86.36) (width 0.25) (layer B.Cu) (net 12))
 (segment (start 142.875 86.36) (end 142.875 96.44) (width 0.25) (layer B.Cu) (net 12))
 (segment (start 142.875 96.44) (end 144.78 98.98) (width 0.25) (layer B.Cu) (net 12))
 (segment (start 161.925 96.44) (end 161.925 95.29) (width 0.4) (layer B.Cu) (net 13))
 (segment (start 161.925 95.29) (end 162.45001 94.76499) (width 0.4) (layer B.Cu) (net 13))
 (segment (start 162.45001 94.76499) (end 162.45001 94.72499) (width 0.4) (layer B.Cu) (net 13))
 (segment (start 162.45001 94.72499) (end 162.56 94.615) (width 0.4) (layer B.Cu) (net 13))
 (segment (start 162.56 94.615) (end 162.56 88.9) (width 0.4) (layer B.Cu) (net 13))
 (segment (start 162.56 88.9) (end 161.67 88.01) (width 0.4) (layer B.Cu) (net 13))
 (segment (start 161.67 88.01) (end 160.05 88.01) (width 0.4) (layer B.Cu) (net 13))
 (segment (start 160.05 80.01) (end 157.56 80.01) (width 0.25) (layer B.Cu) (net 14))
 (segment (start 160.05 84.01) (end 158.97 85.09) (width 0.25) (layer B.Cu) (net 15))
 (segment (start 158.97 85.09) (end 157.56 85.09) (width 0.25) (layer B.Cu) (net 15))
 (segment (start 160.05 92.01) (end 159.43 92.63) (width 0.25) (layer B.Cu) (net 16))
 (segment (start 159.43 92.63) (end 157.48 92.63) (width 0.25) (layer B.Cu) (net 16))
 (segment (start 160.05 82.01) (end 159.51 82.55) (width 0.25) (layer B.Cu) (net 17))
 (segment (start 159.51 82.55) (end 157.56 82.55) (width 0.25) (layer B.Cu) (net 17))
 (segment (start 160.05 86.01) (end 159.28 86.01) (width 0.25) (layer B.Cu) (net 18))
 (segment (start 159.28 86.01) (end 157.66 87.63) (width 0.25) (layer B.Cu) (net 18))
 (segment (start 157.66 87.63) (end 157.56 87.63) (width 0.25) (layer B.Cu) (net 18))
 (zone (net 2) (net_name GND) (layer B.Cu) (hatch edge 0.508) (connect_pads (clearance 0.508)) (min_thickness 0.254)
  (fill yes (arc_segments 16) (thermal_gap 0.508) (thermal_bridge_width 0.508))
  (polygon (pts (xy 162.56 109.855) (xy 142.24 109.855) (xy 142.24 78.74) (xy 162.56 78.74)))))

